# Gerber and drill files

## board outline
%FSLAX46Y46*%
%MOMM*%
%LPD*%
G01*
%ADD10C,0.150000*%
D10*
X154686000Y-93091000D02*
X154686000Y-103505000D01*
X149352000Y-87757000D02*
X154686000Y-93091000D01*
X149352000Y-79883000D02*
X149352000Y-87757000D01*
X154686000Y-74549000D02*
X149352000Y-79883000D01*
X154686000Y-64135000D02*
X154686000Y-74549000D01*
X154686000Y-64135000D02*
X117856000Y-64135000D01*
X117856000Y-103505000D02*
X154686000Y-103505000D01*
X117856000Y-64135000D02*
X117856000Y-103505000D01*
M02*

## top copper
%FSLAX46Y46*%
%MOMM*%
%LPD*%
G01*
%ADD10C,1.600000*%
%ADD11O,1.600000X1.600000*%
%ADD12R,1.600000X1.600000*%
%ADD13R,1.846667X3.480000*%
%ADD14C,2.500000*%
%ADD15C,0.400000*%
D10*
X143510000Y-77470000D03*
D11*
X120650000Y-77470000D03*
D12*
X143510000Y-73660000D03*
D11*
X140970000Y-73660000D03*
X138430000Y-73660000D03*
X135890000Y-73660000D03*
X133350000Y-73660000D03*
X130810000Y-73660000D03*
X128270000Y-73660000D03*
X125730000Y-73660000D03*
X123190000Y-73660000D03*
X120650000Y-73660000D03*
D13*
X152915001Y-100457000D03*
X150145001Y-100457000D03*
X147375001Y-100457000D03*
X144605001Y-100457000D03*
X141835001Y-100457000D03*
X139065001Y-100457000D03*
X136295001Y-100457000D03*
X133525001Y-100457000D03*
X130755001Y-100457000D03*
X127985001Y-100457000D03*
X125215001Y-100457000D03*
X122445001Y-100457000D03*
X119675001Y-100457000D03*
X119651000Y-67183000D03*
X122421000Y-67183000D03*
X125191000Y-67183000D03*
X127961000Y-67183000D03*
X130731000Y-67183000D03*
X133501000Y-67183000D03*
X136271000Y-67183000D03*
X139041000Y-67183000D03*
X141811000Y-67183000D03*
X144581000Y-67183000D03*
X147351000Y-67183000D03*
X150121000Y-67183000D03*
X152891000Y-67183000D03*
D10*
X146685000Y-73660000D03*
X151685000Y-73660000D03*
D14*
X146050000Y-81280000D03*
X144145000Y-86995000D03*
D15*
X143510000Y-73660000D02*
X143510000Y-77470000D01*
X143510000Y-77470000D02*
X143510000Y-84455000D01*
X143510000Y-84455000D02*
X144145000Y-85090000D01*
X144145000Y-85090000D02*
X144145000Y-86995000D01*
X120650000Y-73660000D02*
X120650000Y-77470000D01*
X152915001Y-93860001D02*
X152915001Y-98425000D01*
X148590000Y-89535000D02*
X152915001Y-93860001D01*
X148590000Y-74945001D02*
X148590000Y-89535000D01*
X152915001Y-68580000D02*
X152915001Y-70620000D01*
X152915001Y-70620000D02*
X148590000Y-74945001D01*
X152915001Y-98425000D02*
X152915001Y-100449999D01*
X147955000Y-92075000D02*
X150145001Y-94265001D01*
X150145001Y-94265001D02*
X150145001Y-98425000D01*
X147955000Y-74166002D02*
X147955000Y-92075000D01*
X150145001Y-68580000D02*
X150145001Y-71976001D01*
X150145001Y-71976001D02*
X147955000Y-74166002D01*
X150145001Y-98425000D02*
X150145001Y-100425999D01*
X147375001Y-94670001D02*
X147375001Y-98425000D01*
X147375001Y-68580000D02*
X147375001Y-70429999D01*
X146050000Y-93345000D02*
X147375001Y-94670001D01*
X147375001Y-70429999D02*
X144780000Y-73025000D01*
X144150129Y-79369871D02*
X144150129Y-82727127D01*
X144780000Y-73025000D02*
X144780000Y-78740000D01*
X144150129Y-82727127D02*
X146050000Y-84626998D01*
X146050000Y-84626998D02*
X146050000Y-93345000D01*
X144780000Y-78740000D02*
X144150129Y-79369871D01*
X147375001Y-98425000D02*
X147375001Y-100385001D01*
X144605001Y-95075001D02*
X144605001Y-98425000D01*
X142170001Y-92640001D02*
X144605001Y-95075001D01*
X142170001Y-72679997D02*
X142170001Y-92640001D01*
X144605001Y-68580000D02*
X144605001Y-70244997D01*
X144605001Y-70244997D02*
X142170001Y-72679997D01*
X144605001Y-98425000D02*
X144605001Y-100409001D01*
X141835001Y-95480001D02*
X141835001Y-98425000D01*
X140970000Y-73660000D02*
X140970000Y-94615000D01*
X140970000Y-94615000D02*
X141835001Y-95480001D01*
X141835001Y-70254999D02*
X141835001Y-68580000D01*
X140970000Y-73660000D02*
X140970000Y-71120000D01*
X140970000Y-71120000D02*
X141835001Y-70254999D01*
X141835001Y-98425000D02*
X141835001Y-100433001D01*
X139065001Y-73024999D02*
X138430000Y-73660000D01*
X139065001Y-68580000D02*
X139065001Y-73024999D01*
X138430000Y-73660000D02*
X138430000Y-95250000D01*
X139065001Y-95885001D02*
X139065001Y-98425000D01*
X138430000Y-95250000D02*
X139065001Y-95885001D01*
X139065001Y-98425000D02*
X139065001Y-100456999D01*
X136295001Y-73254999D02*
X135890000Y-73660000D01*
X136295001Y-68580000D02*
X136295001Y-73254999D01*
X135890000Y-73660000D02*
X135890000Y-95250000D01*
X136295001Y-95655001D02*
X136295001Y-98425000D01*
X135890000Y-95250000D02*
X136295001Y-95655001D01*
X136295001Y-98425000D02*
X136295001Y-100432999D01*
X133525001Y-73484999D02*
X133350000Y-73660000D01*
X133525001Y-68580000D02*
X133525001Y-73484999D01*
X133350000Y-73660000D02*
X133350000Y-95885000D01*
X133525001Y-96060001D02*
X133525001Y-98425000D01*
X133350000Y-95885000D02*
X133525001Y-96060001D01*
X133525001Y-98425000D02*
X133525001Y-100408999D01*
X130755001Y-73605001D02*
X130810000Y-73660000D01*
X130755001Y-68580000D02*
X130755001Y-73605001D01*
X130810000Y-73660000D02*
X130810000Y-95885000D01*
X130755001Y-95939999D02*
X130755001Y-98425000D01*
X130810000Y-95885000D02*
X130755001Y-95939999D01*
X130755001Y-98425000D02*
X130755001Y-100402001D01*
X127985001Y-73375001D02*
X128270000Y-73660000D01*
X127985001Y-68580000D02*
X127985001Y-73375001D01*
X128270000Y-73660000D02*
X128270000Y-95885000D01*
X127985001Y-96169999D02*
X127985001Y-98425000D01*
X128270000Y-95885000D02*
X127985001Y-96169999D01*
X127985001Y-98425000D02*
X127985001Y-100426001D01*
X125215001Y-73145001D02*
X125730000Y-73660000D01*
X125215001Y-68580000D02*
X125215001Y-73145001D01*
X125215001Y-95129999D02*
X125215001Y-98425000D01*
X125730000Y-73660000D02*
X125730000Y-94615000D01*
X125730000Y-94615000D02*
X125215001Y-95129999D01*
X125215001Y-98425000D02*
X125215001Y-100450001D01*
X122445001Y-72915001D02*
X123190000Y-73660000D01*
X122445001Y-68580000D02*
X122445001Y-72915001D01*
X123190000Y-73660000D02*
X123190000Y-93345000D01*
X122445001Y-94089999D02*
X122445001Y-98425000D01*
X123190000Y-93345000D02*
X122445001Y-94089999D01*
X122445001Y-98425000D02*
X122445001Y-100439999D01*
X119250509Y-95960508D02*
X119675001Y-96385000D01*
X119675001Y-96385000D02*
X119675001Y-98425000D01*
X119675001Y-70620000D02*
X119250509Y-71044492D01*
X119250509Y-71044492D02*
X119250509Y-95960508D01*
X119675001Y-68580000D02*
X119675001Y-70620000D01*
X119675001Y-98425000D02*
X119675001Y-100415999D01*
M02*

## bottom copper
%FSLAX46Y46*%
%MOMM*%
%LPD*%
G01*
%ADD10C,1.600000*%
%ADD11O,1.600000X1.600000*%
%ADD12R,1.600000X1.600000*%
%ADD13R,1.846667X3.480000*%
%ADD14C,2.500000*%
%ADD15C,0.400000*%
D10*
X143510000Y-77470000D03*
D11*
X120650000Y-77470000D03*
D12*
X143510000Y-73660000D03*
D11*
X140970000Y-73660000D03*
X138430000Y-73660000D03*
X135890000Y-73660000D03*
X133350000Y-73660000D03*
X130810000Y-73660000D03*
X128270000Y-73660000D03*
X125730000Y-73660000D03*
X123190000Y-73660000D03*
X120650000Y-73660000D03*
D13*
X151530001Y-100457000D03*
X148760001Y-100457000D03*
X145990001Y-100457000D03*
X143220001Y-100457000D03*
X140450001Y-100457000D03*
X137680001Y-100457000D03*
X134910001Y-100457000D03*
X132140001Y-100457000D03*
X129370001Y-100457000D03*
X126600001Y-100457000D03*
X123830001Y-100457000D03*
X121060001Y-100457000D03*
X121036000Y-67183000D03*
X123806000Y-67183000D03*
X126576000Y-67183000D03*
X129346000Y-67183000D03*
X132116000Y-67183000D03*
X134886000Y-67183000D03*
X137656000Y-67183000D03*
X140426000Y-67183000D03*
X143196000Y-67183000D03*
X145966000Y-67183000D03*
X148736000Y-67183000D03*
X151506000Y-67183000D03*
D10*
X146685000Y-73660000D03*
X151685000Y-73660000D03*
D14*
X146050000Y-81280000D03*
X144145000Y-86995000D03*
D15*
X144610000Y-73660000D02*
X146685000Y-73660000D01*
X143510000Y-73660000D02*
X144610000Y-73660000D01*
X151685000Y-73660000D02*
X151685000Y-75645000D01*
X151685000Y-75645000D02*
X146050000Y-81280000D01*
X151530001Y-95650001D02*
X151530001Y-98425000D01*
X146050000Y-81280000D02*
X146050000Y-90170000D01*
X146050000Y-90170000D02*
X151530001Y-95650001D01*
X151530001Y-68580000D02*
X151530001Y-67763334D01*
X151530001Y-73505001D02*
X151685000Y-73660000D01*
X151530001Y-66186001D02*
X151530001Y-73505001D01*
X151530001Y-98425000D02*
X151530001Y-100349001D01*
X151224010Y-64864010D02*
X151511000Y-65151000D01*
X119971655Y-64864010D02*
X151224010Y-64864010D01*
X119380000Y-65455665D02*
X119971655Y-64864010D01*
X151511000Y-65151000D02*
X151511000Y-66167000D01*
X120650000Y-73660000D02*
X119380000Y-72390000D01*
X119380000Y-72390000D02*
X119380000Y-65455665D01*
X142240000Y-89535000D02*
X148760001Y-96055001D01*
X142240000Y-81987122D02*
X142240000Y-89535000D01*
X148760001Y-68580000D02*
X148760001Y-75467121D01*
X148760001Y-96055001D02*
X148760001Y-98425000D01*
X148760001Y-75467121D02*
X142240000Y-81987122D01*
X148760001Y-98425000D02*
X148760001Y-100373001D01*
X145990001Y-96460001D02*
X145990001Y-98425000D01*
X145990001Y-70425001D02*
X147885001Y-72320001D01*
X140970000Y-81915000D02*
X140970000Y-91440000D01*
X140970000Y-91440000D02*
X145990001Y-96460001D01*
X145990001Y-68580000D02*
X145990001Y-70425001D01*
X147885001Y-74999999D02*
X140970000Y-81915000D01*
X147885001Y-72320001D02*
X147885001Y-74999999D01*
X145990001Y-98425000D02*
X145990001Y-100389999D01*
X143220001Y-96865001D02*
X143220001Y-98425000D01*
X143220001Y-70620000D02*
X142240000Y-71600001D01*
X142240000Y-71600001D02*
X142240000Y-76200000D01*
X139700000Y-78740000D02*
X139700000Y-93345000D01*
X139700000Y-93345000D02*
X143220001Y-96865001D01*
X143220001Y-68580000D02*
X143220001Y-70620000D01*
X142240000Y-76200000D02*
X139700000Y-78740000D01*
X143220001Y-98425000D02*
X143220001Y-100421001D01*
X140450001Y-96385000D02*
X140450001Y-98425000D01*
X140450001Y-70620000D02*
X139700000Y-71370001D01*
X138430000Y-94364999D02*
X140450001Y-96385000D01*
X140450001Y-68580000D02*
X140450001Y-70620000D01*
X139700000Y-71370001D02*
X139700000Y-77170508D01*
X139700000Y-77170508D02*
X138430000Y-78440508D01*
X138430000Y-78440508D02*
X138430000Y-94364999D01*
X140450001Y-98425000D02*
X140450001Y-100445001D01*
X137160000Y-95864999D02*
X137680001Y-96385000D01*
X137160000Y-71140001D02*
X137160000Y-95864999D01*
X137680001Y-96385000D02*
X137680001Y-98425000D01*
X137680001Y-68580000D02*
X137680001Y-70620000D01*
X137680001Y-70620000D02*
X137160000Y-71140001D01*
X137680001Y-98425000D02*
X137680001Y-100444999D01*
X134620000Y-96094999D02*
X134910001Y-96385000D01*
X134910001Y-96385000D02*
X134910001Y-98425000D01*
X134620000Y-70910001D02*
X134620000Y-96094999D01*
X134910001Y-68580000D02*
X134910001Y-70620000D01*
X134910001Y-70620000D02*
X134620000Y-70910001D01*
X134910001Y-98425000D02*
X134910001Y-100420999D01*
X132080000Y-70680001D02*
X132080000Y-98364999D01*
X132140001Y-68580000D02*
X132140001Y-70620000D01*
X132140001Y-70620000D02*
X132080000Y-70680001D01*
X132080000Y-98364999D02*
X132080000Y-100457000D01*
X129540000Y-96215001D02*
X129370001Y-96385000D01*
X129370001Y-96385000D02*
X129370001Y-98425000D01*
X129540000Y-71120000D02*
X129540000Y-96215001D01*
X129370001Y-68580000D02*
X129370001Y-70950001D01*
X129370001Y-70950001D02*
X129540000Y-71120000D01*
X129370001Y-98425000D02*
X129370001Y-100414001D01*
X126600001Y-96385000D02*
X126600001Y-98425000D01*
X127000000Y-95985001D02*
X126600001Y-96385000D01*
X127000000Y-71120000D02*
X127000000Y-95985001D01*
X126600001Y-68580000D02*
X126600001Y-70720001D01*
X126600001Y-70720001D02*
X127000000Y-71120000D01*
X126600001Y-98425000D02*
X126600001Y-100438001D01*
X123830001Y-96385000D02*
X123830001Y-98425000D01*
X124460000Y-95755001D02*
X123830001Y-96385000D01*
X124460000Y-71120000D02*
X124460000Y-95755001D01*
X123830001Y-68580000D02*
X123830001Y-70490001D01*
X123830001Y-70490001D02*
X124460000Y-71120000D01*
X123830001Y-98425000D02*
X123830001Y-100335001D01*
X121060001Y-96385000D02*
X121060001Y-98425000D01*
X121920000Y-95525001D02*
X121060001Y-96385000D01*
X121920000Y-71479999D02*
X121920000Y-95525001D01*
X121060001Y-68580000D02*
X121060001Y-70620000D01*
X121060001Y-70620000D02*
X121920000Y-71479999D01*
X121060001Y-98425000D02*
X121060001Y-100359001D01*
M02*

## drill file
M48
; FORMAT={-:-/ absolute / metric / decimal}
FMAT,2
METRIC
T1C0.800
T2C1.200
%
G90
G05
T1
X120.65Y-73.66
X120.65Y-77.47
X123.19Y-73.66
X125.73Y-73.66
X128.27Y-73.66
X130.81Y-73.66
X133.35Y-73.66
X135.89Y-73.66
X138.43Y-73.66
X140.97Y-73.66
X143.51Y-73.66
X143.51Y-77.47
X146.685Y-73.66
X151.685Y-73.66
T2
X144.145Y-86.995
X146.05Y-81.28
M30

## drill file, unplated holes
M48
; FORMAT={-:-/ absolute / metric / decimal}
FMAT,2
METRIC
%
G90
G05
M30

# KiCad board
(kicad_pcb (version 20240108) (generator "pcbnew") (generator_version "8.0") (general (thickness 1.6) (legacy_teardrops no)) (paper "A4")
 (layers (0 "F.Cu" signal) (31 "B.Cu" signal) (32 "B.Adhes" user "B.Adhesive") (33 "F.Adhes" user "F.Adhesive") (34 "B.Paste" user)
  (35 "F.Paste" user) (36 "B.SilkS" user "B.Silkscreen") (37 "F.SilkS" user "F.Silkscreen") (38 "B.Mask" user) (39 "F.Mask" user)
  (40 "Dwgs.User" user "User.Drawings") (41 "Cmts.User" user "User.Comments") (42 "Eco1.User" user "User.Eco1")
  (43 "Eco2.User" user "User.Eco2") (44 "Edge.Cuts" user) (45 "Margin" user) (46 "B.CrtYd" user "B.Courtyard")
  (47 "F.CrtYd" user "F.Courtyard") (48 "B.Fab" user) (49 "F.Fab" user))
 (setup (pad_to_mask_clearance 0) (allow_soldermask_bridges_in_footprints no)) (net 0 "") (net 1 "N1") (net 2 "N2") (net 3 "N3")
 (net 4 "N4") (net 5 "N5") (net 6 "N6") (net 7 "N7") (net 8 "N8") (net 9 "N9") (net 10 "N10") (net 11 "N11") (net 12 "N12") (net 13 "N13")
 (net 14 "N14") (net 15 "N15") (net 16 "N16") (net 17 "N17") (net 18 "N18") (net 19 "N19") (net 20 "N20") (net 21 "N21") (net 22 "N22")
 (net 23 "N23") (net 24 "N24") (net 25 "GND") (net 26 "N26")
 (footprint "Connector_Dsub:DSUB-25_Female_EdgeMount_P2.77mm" (layer "F.Cu") (at 136.271 67.183 180)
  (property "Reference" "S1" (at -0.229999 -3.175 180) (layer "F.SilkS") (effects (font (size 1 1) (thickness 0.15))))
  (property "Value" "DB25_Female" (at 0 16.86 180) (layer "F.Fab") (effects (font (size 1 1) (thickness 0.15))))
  (pad "1" smd rect (at 16.62 0 180) (size 1.846667 3.48) (layers "F.Cu" "F.Paste" "F.Mask") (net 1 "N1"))
  (pad "2" smd rect (at 13.85 0 180) (size 1.846667 3.48) (layers "F.Cu" "F.Paste" "F.Mask") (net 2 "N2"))
  (pad "3" smd rect (at 11.08 0 180) (size 1.846667 3.48) (layers "F.Cu" "F.Paste" "F.Mask") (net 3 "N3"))
  (pad "4" smd rect (at 8.31 0 180) (size 1.846667 3.48) (layers "F.Cu" "F.Paste" "F.Mask") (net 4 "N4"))
  (pad "5" smd rect (at 5.54 0 180) (size 1.846667 3.48) (layers "F.Cu" "F.Paste" "F.Mask") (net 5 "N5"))
  (pad "6" smd rect (at 2.77 0 180) (size 1.846667 3.48) (layers "F.Cu" "F.Paste" "F.Mask") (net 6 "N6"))
  (pad "7" smd rect (at 0 0 180) (size 1.846667 3.48) (layers "F.Cu" "F.Paste" "F.Mask") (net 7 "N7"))
  (pad "8" smd rect (at -2.77 0 180) (size 1.846667 3.48) (layers "F.Cu" "F.Paste" "F.Mask") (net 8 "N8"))
  (pad "9" smd rect (at -5.54 0 180) (size 1.846667 3.48) (layers "F.Cu" "F.Paste" "F.Mask") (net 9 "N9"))
  (pad "10" smd rect (at -8.31 0 180) (size 1.846667 3.48) (layers "F.Cu" "F.Paste" "F.Mask") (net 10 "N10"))
  (pad "11" smd rect (at -11.08 0 180) (size 1.846667 3.48) (layers "F.Cu" "F.Paste" "F.Mask") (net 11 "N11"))
  (pad "12" smd rect (at -13.85 0 180) (size 1.846667 3.48) (layers "F.Cu" "F.Paste" "F.Mask") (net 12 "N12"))
  (pad "13" smd rect (at -16.62 0 180) (size 1.846667 3.48) (layers "F.Cu" "F.Paste" "F.Mask") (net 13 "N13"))
  (pad "14" smd rect (at 15.235 0 180) (size 1.846667 3.48) (layers "B.Cu" "B.Paste" "B.Mask") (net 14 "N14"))
  (pad "15" smd rect (at 12.465 0 180) (size 1.846667 3.48) (layers "B.Cu" "B.Paste" "B.Mask") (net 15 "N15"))
  (pad "16" smd rect (at 9.695 0 180) (size 1.846667 3.48) (layers "B.Cu" "B.Paste" "B.Mask") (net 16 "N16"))
  (pad "17" smd rect (at 6.925 0 180) (size 1.846667 3.48) (layers "B.Cu" "B.Paste" "B.Mask") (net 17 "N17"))
  (pad "18" smd rect (at 4.155 0 180) (size 1.846667 3.48) (layers "B.Cu" "B.Paste" "B.Mask") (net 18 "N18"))
  (pad "19" smd rect (at 1.385 0 180) (size 1.846667 3.48) (layers "B.Cu" "B.Paste" "B.Mask") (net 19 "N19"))
  (pad "20" smd rect (at -1.385 0 180) (size 1.846667 3.48) (layers "B.Cu" "B.Paste" "B.Mask") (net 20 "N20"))
  (pad "21" smd rect (at -4.155 0 180) (size 1.846667 3.48) (layers "B.Cu" "B.Paste" "B.Mask") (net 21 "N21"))
  (pad "22" smd rect (at -6.925 0 180) (size 1.846667 3.48) (layers "B.Cu" "B.Paste" "B.Mask") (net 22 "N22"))
  (pad "23" smd rect (at -9.695 0 180) (size 1.846667 3.48) (layers "B.Cu" "B.Paste" "B.Mask") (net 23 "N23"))
  (pad "24" smd rect (at -12.465 0 180) (size 1.846667 3.48) (layers "B.Cu" "B.Paste" "B.Mask") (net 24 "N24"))
  (pad "25" smd rect (at -15.235 0 180) (size 1.846667 3.48) (layers "B.Cu" "B.Paste" "B.Mask") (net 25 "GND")))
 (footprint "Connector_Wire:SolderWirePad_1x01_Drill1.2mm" (layer "F.Cu") (at 146.05 81.28)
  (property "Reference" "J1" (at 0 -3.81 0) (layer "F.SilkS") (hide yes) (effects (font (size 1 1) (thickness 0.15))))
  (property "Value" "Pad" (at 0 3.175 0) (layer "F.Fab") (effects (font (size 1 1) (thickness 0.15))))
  (pad "1" thru_hole circle (at 0 0) (size 2.5 2.5) (drill 1.2) (layers "*.Cu" "*.Mask") (remove_unused_layers no) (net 25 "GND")))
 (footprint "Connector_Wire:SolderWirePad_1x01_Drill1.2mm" (layer "F.Cu") (at 144.145 86.995)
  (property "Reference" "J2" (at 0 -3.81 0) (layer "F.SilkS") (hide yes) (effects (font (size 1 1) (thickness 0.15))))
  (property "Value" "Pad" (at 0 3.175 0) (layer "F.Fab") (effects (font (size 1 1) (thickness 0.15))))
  (pad "1" thru_hole circle (at 0 0) (size 2.5 2.5) (drill 1.2) (layers "*.Cu" "*.Mask") (remove_unused_layers no) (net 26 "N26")))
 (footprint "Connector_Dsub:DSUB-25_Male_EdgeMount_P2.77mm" (layer "F.Cu") (at 136.295001 100.457)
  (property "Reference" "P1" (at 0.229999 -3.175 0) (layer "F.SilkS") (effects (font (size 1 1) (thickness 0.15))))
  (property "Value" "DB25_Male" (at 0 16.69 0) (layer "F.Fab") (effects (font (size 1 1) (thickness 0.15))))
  (pad "1" smd rect (at -16.62 0) (size 1.846667 3.48) (layers "F.Cu" "F.Paste" "F.Mask") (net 1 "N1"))
  (pad "2" smd rect (at -13.85 0) (size 1.846667 3.48) (layers "F.Cu" "F.Paste" "F.Mask") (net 2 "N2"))
  (pad "3" smd rect (at -11.08 0) (size 1.846667 3.48) (layers "F.Cu" "F.Paste" "F.Mask") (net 3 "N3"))
  (pad "4" smd rect (at -8.31 0) (size 1.846667 3.48) (layers "F.Cu" "F.Paste" "F.Mask") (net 4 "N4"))
  (pad "5" smd rect (at -5.54 0) (size 1.846667 3.48) (layers "F.Cu" "F.Paste" "F.Mask") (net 5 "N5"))
  (pad "6" smd rect (at -2.77 0) (size 1.846667 3.48) (layers "F.Cu" "F.Paste" "F.Mask") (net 6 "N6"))
  (pad "7" smd rect (at 0 0) (size 1.846667 3.48) (layers "F.Cu" "F.Paste" "F.Mask") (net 7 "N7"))
  (pad "8" smd rect (at 2.77 0) (size 1.846667 3.48) (layers "F.Cu" "F.Paste" "F.Mask") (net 8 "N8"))
  (pad "9" smd rect (at 5.54 0) (size 1.846667 3.48) (layers "F.Cu" "F.Paste" "F.Mask") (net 9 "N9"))
  (pad "10" smd rect (at 8.31 0) (size 1.846667 3.48) (layers "F.Cu" "F.Paste" "F.Mask") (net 10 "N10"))
  (pad "11" smd rect (at 11.08 0) (size 1.846667 3.48) (layers "F.Cu" "F.Paste" "F.Mask") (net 11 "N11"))
  (pad "12" smd rect (at 13.85 0) (size 1.846667 3.48) (layers "F.Cu" "F.Paste" "F.Mask") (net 12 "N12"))
  (pad "13" smd rect (at 16.62 0) (size 1.846667 3.48) (layers "F.Cu" "F.Paste" "F.Mask") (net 13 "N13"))
  (pad "14" smd rect (at -15.235 0) (size 1.846667 3.48) (layers "B.Cu" "B.Paste" "B.Mask") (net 14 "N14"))
  (pad "15" smd rect (at -12.465 0) (size 1.846667 3.48) (layers "B.Cu" "B.Paste" "B.Mask") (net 15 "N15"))
  (pad "16" smd rect (at -9.695 0) (size 1.846667 3.48) (layers "B.Cu" "B.Paste" "B.Mask") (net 16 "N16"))
  (pad "17" smd rect (at -6.925 0) (size 1.846667 3.48) (layers "B.Cu" "B.Paste" "B.Mask") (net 17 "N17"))
  (pad "18" smd rect (at -4.155 0) (size 1.846667 3.48) (layers "B.Cu" "B.Paste" "B.Mask") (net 18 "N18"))
  (pad "19" smd rect (at -1.385 0) (size 1.846667 3.48) (layers "B.Cu" "B.Paste" "B.Mask") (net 19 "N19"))
  (pad "20" smd rect (at 1.385 0) (size 1.846667 3.48) (layers "B.Cu" "B.Paste" "B.Mask") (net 20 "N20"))
  (pad "21" smd rect (at 4.155 0) (size 1.846667 3.48) (layers "B.Cu" "B.Paste" "B.Mask") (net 21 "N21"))
  (pad "22" smd rect (at 6.925 0) (size 1.846667 3.48) (layers "B.Cu" "B.Paste" "B.Mask") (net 22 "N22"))
  (pad "23" smd rect (at 9.695 0) (size 1.846667 3.48) (layers "B.Cu" "B.Paste" "B.Mask") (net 23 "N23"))
  (pad "24" smd rect (at 12.465 0) (size 1.846667 3.48) (layers "B.Cu" "B.Paste" "B.Mask") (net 24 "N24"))
  (pad "25" smd rect (at 15.235 0) (size 1.846667 3.48) (layers "B.Cu" "B.Paste" "B.Mask") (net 25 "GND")))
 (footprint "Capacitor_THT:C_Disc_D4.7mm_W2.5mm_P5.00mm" (layer "B.Cu") (at 146.685 73.66)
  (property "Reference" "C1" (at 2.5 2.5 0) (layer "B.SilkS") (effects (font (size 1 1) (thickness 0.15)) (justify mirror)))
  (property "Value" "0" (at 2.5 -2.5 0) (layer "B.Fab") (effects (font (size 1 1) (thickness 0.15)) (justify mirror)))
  (pad "1" thru_hole circle (at 0 0) (size 1.6 1.6) (drill 0.8) (layers "*.Cu" "*.Mask") (remove_unused_layers no) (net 26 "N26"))
  (pad "2" thru_hole circle (at 5 0) (size 1.6 1.6) (drill 0.8) (layers "*.Cu" "*.Mask") (remove_unused_layers no) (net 25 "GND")))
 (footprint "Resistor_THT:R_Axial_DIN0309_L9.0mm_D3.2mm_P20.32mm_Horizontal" (layer "B.Cu") (at 143.51 77.47 180)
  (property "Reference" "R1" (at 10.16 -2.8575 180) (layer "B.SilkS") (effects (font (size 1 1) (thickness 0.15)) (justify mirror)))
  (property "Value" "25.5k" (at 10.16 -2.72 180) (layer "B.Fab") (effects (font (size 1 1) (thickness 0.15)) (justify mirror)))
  (pad "1" thru_hole circle (at 0 0 180) (size 1.6 1.6) (drill 0.8) (layers "*.Cu" "*.Mask") (remove_unused_layers no) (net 26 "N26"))
  (pad "2" thru_hole oval (at 22.86 0 180) (size 1.6 1.6) (drill 0.8) (layers "*.Cu" "*.Mask") (remove_unused_layers no) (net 25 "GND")))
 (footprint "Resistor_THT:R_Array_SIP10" (layer "B.Cu") (at 143.51 73.66 180)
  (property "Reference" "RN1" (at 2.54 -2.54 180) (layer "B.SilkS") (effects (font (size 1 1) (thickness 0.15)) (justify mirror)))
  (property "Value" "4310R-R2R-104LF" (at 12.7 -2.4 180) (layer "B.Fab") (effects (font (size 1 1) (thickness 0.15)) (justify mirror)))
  (pad "1" thru_hole rect (at 0 0 180) (size 1.6 1.6) (drill 0.8) (layers "*.Cu" "*.Mask") (remove_unused_layers no) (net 26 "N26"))
  (pad "2" thru_hole oval (at 2.54 0 180) (size 1.6 1.6) (drill 0.8) (layers "*.Cu" "*.Mask") (remove_unused_layers no) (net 9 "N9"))
  (pad "3" thru_hole oval (at 5.08 0 180) (size 1.6 1.6) (drill 0.8) (layers "*.Cu" "*.Mask") (remove_unused_layers no) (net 8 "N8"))
  (pad "4" thru_hole oval (at 7.62 0 180) (size 1.6 1.6) (drill 0.8) (layers "*.Cu" "*.Mask") (remove_unused_layers no) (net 7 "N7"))
  (pad "5" thru_hole oval (at 10.16 0 180) (size 1.6 1.6) (drill 0.8) (layers "*.Cu" "*.Mask") (remove_unused_layers no) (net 6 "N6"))
  (pad "6" thru_hole oval (at 12.7 0 180) (size 1.6 1.6) (drill 0.8) (layers "*.Cu" "*.Mask") (remove_unused_layers no) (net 5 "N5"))
  (pad "7" thru_hole oval (at 15.24 0 180) (size 1.6 1.6) (drill 0.8) (layers "*.Cu" "*.Mask") (remove_unused_layers no) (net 4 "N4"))
  (pad "8" thru_hole oval (at 17.78 0 180) (size 1.6 1.6) (drill 0.8) (layers "*.Cu" "*.Mask") (remove_unused_layers no) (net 3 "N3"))
  (pad "9" thru_hole oval (at 20.32 0 180) (size 1.6 1.6) (drill 0.8) (layers "*.Cu" "*.Mask") (remove_unused_layers no) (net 2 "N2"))
  (pad "10" thru_hole oval (at 22.86 0 180) (size 1.6 1.6) (drill 0.8) (layers "*.Cu" "*.Mask") (remove_unused_layers no) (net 25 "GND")))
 (gr_line (start 154.686 64.135) (end 154.686 74.549) (stroke (width 0.15) (type solid)) (layer "Edge.Cuts"))
 (gr_line (start 149.352 79.883) (end 149.352 87.757) (stroke (width 0.15) (type solid)) (layer "Edge.Cuts"))
 (gr_line (start 154.686 64.135) (end 117.856 64.135) (stroke (width 0.15) (type solid)) (layer "Edge.Cuts"))
 (gr_line (start 117.856 64.135) (end 117.856 103.505) (stroke (width 0.15) (type solid)) (layer "Edge.Cuts"))
 (gr_line (start 149.352 87.757) (end 154.686 93.091) (stroke (width 0.15) (type solid)) (layer "Edge.Cuts"))
 (gr_line (start 117.856 103.505) (end 154.686 103.505) (stroke (width 0.15) (type solid)) (layer "Edge.Cuts"))
 (gr_line (start 154.686 74.549) (end 149.352 79.883) (stroke (width 0.15) (type solid)) (layer "Edge.Cuts"))
 (gr_line (start 154.686 93.091) (end 154.686 103.505) (stroke (width 0.15) (type solid)) (layer "Edge.Cuts"))
 (segment (start 143.51 73.66) (end 143.51 77.47) (width 0.4) (layer "F.Cu") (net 26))
 (segment (start 143.51 84.455) (end 144.145 85.09) (width 0.4) (layer "F.Cu") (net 26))
 (segment (start 143.51 77.47) (end 143.51 84.455) (width 0.4) (layer "F.Cu") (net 26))
 (segment (start 144.145 85.09) (end 144.145 86.995) (width 0.4) (layer "F.Cu") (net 26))
 (segment (start 144.61 73.66) (end 146.685 73.66) (width 0.4) (layer "B.Cu") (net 26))
 (segment (start 143.51 73.66) (end 144.61 73.66) (width 0.4) (layer "B.Cu") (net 26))
 (segment (start 120.65 73.66) (end 120.65 77.47) (width 0.4) (layer "F.Cu") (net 25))
 (segment (start 119.38 65.455665) (end 119.971655 64.86401) (width 0.4) (layer "B.Cu") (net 25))
 (segment (start 151.530001 98.425) (end 151.530001 100.349001) (width 0.4) (layer "B.Cu") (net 25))
 (segment (start 120.65 73.66) (end 119.38 72.39) (width 0.4) (layer "B.Cu") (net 25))
 (segment (start 146.05 81.28) (end 146.05 90.17) (width 0.4) (layer "B.Cu") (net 25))
 (segment (start 151.530001 73.505001) (end 151.685 73.66) (width 0.4) (layer "B.Cu") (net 25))
 (segment (start 151.22401 64.86401) (end 151.511 65.151) (width 0.4) (layer "B.Cu") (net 25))
 (segment (start 119.971655 64.86401) (end 151.22401 64.86401) (width 0.4) (layer "B.Cu") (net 25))
 (segment (start 146.05 90.17) (end 151.530001 95.650001) (width 0.4) (layer "B.Cu") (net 25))
 (segment (start 151.530001 66.186001) (end 151.530001 73.505001) (width 0.4) (layer "B.Cu") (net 25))
 (segment (start 151.530001 68.58) (end 151.530001 67.763334) (width 0.4) (layer "B.Cu") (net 25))
 (segment (start 119.38 72.39) (end 119.38 65.455665) (width 0.4) (layer "B.Cu") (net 25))
 (segment (start 151.511 65.151) (end 151.511 66.167) (width 0.4) (layer "B.Cu") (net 25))
 (segment (start 151.530001 95.650001) (end 151.530001 98.425) (width 0.4) (layer "B.Cu") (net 25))
 (segment (start 151.685 73.66) (end 151.685 75.645) (width 0.4) (layer "B.Cu") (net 25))
 (segment (start 151.685 75.645) (end 146.05 81.28) (width 0.4) (layer "B.Cu") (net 25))
 (segment (start 148.760001 98.425) (end 148.760001 100.373001) (width 0.4) (layer "B.Cu") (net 24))
 (segment (start 142.24 89.535) (end 148.760001 96.055001) (width 0.4) (layer "B.Cu") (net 24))
 (segment (start 148.760001 75.467121) (end 142.24 81.987122) (width 0.4) (layer "B.Cu") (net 24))
 (segment (start 148.760001 96.055001) (end 148.760001 98.425) (width 0.4) (layer "B.Cu") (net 24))
 (segment (start 142.24 81.987122) (end 142.24 89.535) (width 0.4) (layer "B.Cu") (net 24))
 (segment (start 148.760001 68.58) (end 148.760001 75.467121) (width 0.4) (layer "B.Cu") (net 24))
 (segment (start 147.885001 74.999999) (end 140.97 81.915) (width 0.4) (layer "B.Cu") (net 23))
 (segment (start 140.97 81.915) (end 140.97 91.44) (width 0.4) (layer "B.Cu") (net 23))
 (segment (start 140.97 91.44) (end 145.990001 96.460001) (width 0.4) (layer "B.Cu") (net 23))
 (segment (start 145.990001 70.425001) (end 147.885001 72.320001) (width 0.4) (layer "B.Cu") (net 23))
 (segment (start 145.990001 98.425) (end 145.990001 100.389999) (width 0.4) (layer "B.Cu") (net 23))
 (segment (start 145.990001 68.58) (end 145.990001 70.425001) (width 0.4) (layer "B.Cu") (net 23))
 (segment (start 147.885001 72.320001) (end 147.885001 74.999999) (width 0.4) (layer "B.Cu") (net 23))
 (segment (start 145.990001 96.460001) (end 145.990001 98.425) (width 0.4) (layer "B.Cu") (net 23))
 (segment (start 143.220001 96.865001) (end 143.220001 98.425) (width 0.4) (layer "B.Cu") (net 22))
 (segment (start 139.7 78.74) (end 139.7 93.345) (width 0.4) (layer "B.Cu") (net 22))
 (segment (start 143.220001 68.58) (end 143.220001 70.62) (width 0.4) (layer "B.Cu") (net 22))
 (segment (start 139.7 93.345) (end 143.220001 96.865001) (width 0.4) (layer "B.Cu") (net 22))
 (segment (start 142.24 76.2) (end 139.7 78.74) (width 0.4) (layer "B.Cu") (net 22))
 (segment (start 142.24 71.600001) (end 142.24 76.2) (width 0.4) (layer "B.Cu") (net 22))
 (segment (start 143.220001 70.62) (end 142.24 71.600001) (width 0.4) (layer "B.Cu") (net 22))
 (segment (start 143.220001 98.425) (end 143.220001 100.421001) (width 0.4) (layer "B.Cu") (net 22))
 (segment (start 140.450001 70.62) (end 139.7 71.370001) (width 0.4) (layer "B.Cu") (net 21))
 (segment (start 139.7 71.370001) (end 139.7 77.170508) (width 0.4) (layer "B.Cu") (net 21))
 (segment (start 139.7 77.170508) (end 138.43 78.440508) (width 0.4) (layer "B.Cu") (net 21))
 (segment (start 138.43 94.364999) (end 140.450001 96.385) (width 0.4) (layer "B.Cu") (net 21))
 (segment (start 138.43 78.440508) (end 138.43 94.364999) (width 0.4) (layer "B.Cu") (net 21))
 (segment (start 140.450001 98.425) (end 140.450001 100.445001) (width 0.4) (layer "B.Cu") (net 21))
 (segment (start 140.450001 96.385) (end 140.450001 98.425) (width 0.4) (layer "B.Cu") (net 21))
 (segment (start 140.450001 68.58) (end 140.450001 70.62) (width 0.4) (layer "B.Cu") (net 21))
 (segment (start 137.16 71.140001) (end 137.16 95.864999) (width 0.4) (layer "B.Cu") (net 20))
 (segment (start 137.680001 98.425) (end 137.680001 100.444999) (width 0.4) (layer "B.Cu") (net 20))
 (segment (start 137.16 95.864999) (end 137.680001 96.385) (width 0.4) (layer "B.Cu") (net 20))
 (segment (start 137.680001 96.385) (end 137.680001 98.425) (width 0.4) (layer "B.Cu") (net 20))
 (segment (start 137.680001 68.58) (end 137.680001 70.62) (width 0.4) (layer "B.Cu") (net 20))
 (segment (start 137.680001 70.62) (end 137.16 71.140001) (width 0.4) (layer "B.Cu") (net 20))
 (segment (start 134.62 96.094999) (end 134.910001 96.385) (width 0.4) (layer "B.Cu") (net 19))
 (segment (start 134.910001 70.62) (end 134.62 70.910001) (width 0.4) (layer "B.Cu") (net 19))
 (segment (start 134.910001 68.58) (end 134.910001 70.62) (width 0.4) (layer "B.Cu") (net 19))
 (segment (start 134.910001 98.425) (end 134.910001 100.420999) (width 0.4) (layer "B.Cu") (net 19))
 (segment (start 134.910001 96.385) (end 134.910001 98.425) (width 0.4) (layer "B.Cu") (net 19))
 (segment (start 134.62 70.910001) (end 134.62 96.094999) (width 0.4) (layer "B.Cu") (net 19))
 (segment (start 132.08 70.680001) (end 132.08 98.364999) (width 0.4) (layer "B.Cu") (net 18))
 (segment (start 132.140001 68.58) (end 132.140001 70.62) (width 0.4) (layer "B.Cu") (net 18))
 (segment (start 132.08 98.364999) (end 132.08 100.457) (width 0.4) (layer "B.Cu") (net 18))
 (segment (start 132.140001 70.62) (end 132.08 70.680001) (width 0.4) (layer "B.Cu") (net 18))
 (segment (start 129.370001 98.425) (end 129.370001 100.414001) (width 0.4) (layer "B.Cu") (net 17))
 (segment (start 129.370001 68.58) (end 129.370001 70.950001) (width 0.4) (layer "B.Cu") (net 17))
 (segment (start 129.370001 70.950001) (end 129.54 71.12) (width 0.4) (layer "B.Cu") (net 17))
 (segment (start 129.370001 96.385) (end 129.370001 98.425) (width 0.4) (layer "B.Cu") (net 17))
 (segment (start 129.54 96.215001) (end 129.370001 96.385) (width 0.4) (layer "B.Cu") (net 17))
 (segment (start 129.54 71.12) (end 129.54 96.215001) (width 0.4) (layer "B.Cu") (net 17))
 (segment (start 127 95.985001) (end 126.600001 96.385) (width 0.4) (layer "B.Cu") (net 16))
 (segment (start 126.600001 98.425) (end 126.600001 100.438001) (width 0.4) (layer "B.Cu") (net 16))
 (segment (start 126.600001 68.58) (end 126.600001 70.720001) (width 0.4) (layer "B.Cu") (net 16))
 (segment (start 126.600001 70.720001) (end 127 71.12) (width 0.4) (layer "B.Cu") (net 16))
 (segment (start 126.600001 96.385) (end 126.600001 98.425) (width 0.4) (layer "B.Cu") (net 16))
 (segment (start 127 71.12) (end 127 95.985001) (width 0.4) (layer "B.Cu") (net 16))
 (segment (start 123.830001 70.490001) (end 124.46 71.12) (width 0.4) (layer "B.Cu") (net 15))
 (segment (start 124.46 95.755001) (end 123.830001 96.385) (width 0.4) (layer "B.Cu") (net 15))
 (segment (start 123.830001 98.425) (end 123.830001 100.335001) (width 0.4) (layer "B.Cu") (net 15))
 (segment (start 123.830001 96.385) (end 123.830001 98.425) (width 0.4) (layer "B.Cu") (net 15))
 (segment (start 123.830001 68.58) (end 123.830001 70.490001) (width 0.4) (layer "B.Cu") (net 15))
 (segment (start 124.46 71.12) (end 124.46 95.755001) (width 0.4) (layer "B.Cu") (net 15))
 (segment (start 121.92 71.479999) (end 121.92 95.525001) (width 0.4) (layer "B.Cu") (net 14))
 (segment (start 121.060001 68.58) (end 121.060001 70.62) (width 0.4) (layer "B.Cu") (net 14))
 (segment (start 121.060001 96.385) (end 121.060001 98.425) (width 0.4) (layer "B.Cu") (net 14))
 (segment (start 121.92 95.525001) (end 121.060001 96.385) (width 0.4) (layer "B.Cu") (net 14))
 (segment (start 121.060001 98.425) (end 121.060001 100.359001) (width 0.4) (layer "B.Cu") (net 14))
 (segment (start 121.060001 70.62) (end 121.92 71.479999) (width 0.4) (layer "B.Cu") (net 14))
 (segment (start 152.915001 98.425) (end 152.915001 100.449999) (width 0.4) (layer "F.Cu") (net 13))
 (segment (start 148.59 89.535) (end 152.915001 93.860001) (width 0.4) (layer "F.Cu") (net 13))
 (segment (start 148.59 74.945001) (end 148.59 89.535) (width 0.4) (layer "F.Cu") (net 13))
 (segment (start 152.915001 93.860001) (end 152.915001 98.425) (width 0.4) (layer "F.Cu") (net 13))
 (segment (start 152.915001 70.62) (end 148.59 74.945001) (width 0.4) (layer "F.Cu") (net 13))
 (segment (start 152.915001 68.58) (end 152.915001 70.62) (width 0.4) (layer "F.Cu") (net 13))
 (segment (start 150.145001 94.265001) (end 150.145001 98.425) (width 0.4) (layer "F.Cu") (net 12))
 (segment (start 150.145001 68.58) (end 150.145001 71.976001) (width 0.4) (layer "F.Cu") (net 12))
 (segment (start 150.145001 71.976001) (end 147.955 74.166002) (width 0.4) (layer "F.Cu") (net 12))
 (segment (start 147.955 74.166002) (end 147.955 92.075) (width 0.4) (layer "F.Cu") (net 12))
 (segment (start 147.955 92.075) (end 150.145001 94.265001) (width 0.4) (layer "F.Cu") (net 12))
 (segment (start 150.145001 98.425) (end 150.145001 100.425999) (width 0.4) (layer "F.Cu") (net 12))
 (segment (start 144.150129 82.727127) (end 146.05 84.626998) (width 0.4) (layer "F.Cu") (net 11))
 (segment (start 147.375001 98.425) (end 147.375001 100.385001) (width 0.4) (layer "F.Cu") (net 11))
 (segment (start 144.150129 79.369871) (end 144.150129 82.727127) (width 0.4) (layer "F.Cu") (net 11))
 (segment (start 146.05 93.345) (end 147.375001 94.670001) (width 0.4) (layer "F.Cu") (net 11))
 (segment (start 147.375001 68.58) (end 147.375001 70.429999) (width 0.4) (layer "F.Cu") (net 11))
 (segment (start 147.375001 70.429999) (end 144.78 73.025) (width 0.4) (layer "F.Cu") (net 11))
 (segment (start 144.78 78.74) (end 144.150129 79.369871) (width 0.4) (layer "F.Cu") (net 11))
 (segment (start 146.05 84.626998) (end 146.05 93.345) (width 0.4) (layer "F.Cu") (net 11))
 (segment (start 147.375001 94.670001) (end 147.375001 98.425) (width 0.4) (layer "F.Cu") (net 11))
 (segment (start 144.78 73.025) (end 144.78 78.74) (width 0.4) (layer "F.Cu") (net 11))
 (segment (start 142.170001 92.640001) (end 144.605001 95.075001) (width 0.4) (layer "F.Cu") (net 10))
 (segment (start 144.605001 68.58) (end 144.605001 70.244997) (width 0.4) (layer "F.Cu") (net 10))
 (segment (start 142.170001 72.679997) (end 142.170001 92.640001) (width 0.4) (layer "F.Cu") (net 10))
 (segment (start 144.605001 70.244997) (end 142.170001 72.679997) (width 0.4) (layer "F.Cu") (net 10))
 (segment (start 144.605001 95.075001) (end 144.605001 98.425) (width 0.4) (layer "F.Cu") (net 10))
 (segment (start 144.605001 98.425) (end 144.605001 100.409001) (width 0.4) (layer "F.Cu") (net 10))
 (segment (start 140.97 71.12) (end 141.835001 70.254999) (width 0.4) (layer "F.Cu") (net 9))
 (segment (start 141.835001 95.480001) (end 141.835001 98.425) (width 0.4) (layer "F.Cu") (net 9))
 (segment (start 140.97 73.66) (end 140.97 71.12) (width 0.4) (layer "F.Cu") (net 9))
 (segment (start 141.835001 98.425) (end 141.835001 100.433001) (width 0.4) (layer "F.Cu") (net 9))
 (segment (start 140.97 73.66) (end 140.97 94.615) (width 0.4) (layer "F.Cu") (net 9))
 (segment (start 141.835001 70.254999) (end 141.835001 68.58) (width 0.4) (layer "F.Cu") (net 9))
 (segment (start 140.97 94.615) (end 141.835001 95.480001) (width 0.4) (layer "F.Cu") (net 9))
 (segment (start 139.065001 68.58) (end 139.065001 73.024999) (width 0.4) (layer "F.Cu") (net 8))
 (segment (start 139.065001 98.425) (end 139.065001 100.456999) (width 0.4) (layer "F.Cu") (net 8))
 (segment (start 139.065001 95.885001) (end 139.065001 98.425) (width 0.4) (layer "F.Cu") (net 8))
 (segment (start 139.065001 73.024999) (end 138.43 73.66) (width 0.4) (layer "F.Cu") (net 8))
 (segment (start 138.43 95.25) (end 139.065001 95.885001) (width 0.4) (layer "F.Cu") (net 8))
 (segment (start 138.43 73.66) (end 138.43 95.25) (width 0.4) (layer "F.Cu") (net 8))
 (segment (start 136.295001 68.58) (end 136.295001 73.254999) (width 0.4) (layer "F.Cu") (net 7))
 (segment (start 136.295001 73.254999) (end 135.89 73.66) (width 0.4) (layer "F.Cu") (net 7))
 (segment (start 136.295001 95.655001) (end 136.295001 98.425) (width 0.4) (layer "F.Cu") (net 7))
 (segment (start 136.295001 98.425) (end 136.295001 100.432999) (width 0.4) (layer "F.Cu") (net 7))
 (segment (start 135.89 73.66) (end 135.89 95.25) (width 0.4) (layer "F.Cu") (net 7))
 (segment (start 135.89 95.25) (end 136.295001 95.655001) (width 0.4) (layer "F.Cu") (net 7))
 (segment (start 133.525001 73.484999) (end 133.35 73.66) (width 0.4) (layer "F.Cu") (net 6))
 (segment (start 133.35 73.66) (end 133.35 95.885) (width 0.4) (layer "F.Cu") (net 6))
 (segment (start 133.35 95.885) (end 133.525001 96.060001) (width 0.4) (layer "F.Cu") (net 6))
 (segment (start 133.525001 96.060001) (end 133.525001 98.425) (width 0.4) (layer "F.Cu") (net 6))
 (segment (start 133.525001 98.425) (end 133.525001 100.408999) (width 0.4) (layer "F.Cu") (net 6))
 (segment (start 133.525001 68.58) (end 133.525001 73.484999) (width 0.4) (layer "F.Cu") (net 6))
 (segment (start 130.81 95.885) (end 130.755001 95.939999) (width 0.4) (layer "F.Cu") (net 5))
 (segment (start 130.755001 98.425) (end 130.755001 100.402001) (width 0.4) (layer "F.Cu") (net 5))
 (segment (start 130.755001 95.939999) (end 130.755001 98.425) (width 0.4) (layer "F.Cu") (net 5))
 (segment (start 130.81 73.66) (end 130.81 95.885) (width 0.4) (layer "F.Cu") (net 5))
 (segment (start 130.755001 68.58) (end 130.755001 73.605001) (width 0.4) (layer "F.Cu") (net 5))
 (segment (start 130.755001 73.605001) (end 130.81 73.66) (width 0.4) (layer "F.Cu") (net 5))
 (segment (start 127.985001 73.375001) (end 128.27 73.66) (width 0.4) (layer "F.Cu") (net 4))
 (segment (start 128.27 73.66) (end 128.27 95.885) (width 0.4) (layer "F.Cu") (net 4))
 (segment (start 127.985001 96.169999) (end 127.985001 98.425) (width 0.4) (layer "F.Cu") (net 4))
 (segment (start 127.985001 68.58) (end 127.985001 73.375001) (width 0.4) (layer "F.Cu") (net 4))
 (segment (start 127.985001 98.425) (end 127.985001 100.426001) (width 0.4) (layer "F.Cu") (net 4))
 (segment (start 128.27 95.885) (end 127.985001 96.169999) (width 0.4) (layer "F.Cu") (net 4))
 (segment (start 125.215001 73.145001) (end 125.73 73.66) (width 0.4) (layer "F.Cu") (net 3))
 (segment (start 125.215001 98.425) (end 125.215001 100.450001) (width 0.4) (layer "F.Cu") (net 3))
 (segment (start 125.73 94.615) (end 125.215001 95.129999) (width 0.4) (layer "F.Cu") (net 3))
 (segment (start 125.215001 68.58) (end 125.215001 73.145001) (width 0.4) (layer "F.Cu") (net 3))
 (segment (start 125.73 73.66) (end 125.73 94.615) (width 0.4) (layer "F.Cu") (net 3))
 (segment (start 125.215001 95.129999) (end 125.215001 98.425) (width 0.4) (layer "F.Cu") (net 3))
 (segment (start 122.445001 98.425) (end 122.445001 100.439999) (width 0.4) (layer "F.Cu") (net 2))
 (segment (start 123.19 73.66) (end 123.19 93.345) (width 0.4) (layer "F.Cu") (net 2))
 (segment (start 122.445001 94.089999) (end 122.445001 98.425) (width 0.4) (layer "F.Cu") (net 2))
 (segment (start 122.445001 72.915001) (end 123.19 73.66) (width 0.4) (layer "F.Cu") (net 2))
 (segment (start 123.19 93.345) (end 122.445001 94.089999) (width 0.4) (layer "F.Cu") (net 2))
 (segment (start 122.445001 68.58) (end 122.445001 72.915001) (width 0.4) (layer "F.Cu") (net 2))
 (segment (start 119.675001 98.425) (end 119.675001 100.415999) (width 0.4) (layer "F.Cu") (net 1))
 (segment (start 119.250509 71.044492) (end 119.250509 95.960508) (width 0.4) (layer "F.Cu") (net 1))
 (segment (start 119.675001 96.385) (end 119.675001 98.425) (width 0.4) (layer "F.Cu") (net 1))
 (segment (start 119.250509 95.960508) (end 119.675001 96.385) (width 0.4) (layer "F.Cu") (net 1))
 (segment (start 119.675001 70.62) (end 119.250509 71.044492) (width 0.4) (layer "F.Cu") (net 1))
 (segment (start 119.675001 68.58) (end 119.675001 70.62) (width 0.4) (layer "F.Cu") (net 1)))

